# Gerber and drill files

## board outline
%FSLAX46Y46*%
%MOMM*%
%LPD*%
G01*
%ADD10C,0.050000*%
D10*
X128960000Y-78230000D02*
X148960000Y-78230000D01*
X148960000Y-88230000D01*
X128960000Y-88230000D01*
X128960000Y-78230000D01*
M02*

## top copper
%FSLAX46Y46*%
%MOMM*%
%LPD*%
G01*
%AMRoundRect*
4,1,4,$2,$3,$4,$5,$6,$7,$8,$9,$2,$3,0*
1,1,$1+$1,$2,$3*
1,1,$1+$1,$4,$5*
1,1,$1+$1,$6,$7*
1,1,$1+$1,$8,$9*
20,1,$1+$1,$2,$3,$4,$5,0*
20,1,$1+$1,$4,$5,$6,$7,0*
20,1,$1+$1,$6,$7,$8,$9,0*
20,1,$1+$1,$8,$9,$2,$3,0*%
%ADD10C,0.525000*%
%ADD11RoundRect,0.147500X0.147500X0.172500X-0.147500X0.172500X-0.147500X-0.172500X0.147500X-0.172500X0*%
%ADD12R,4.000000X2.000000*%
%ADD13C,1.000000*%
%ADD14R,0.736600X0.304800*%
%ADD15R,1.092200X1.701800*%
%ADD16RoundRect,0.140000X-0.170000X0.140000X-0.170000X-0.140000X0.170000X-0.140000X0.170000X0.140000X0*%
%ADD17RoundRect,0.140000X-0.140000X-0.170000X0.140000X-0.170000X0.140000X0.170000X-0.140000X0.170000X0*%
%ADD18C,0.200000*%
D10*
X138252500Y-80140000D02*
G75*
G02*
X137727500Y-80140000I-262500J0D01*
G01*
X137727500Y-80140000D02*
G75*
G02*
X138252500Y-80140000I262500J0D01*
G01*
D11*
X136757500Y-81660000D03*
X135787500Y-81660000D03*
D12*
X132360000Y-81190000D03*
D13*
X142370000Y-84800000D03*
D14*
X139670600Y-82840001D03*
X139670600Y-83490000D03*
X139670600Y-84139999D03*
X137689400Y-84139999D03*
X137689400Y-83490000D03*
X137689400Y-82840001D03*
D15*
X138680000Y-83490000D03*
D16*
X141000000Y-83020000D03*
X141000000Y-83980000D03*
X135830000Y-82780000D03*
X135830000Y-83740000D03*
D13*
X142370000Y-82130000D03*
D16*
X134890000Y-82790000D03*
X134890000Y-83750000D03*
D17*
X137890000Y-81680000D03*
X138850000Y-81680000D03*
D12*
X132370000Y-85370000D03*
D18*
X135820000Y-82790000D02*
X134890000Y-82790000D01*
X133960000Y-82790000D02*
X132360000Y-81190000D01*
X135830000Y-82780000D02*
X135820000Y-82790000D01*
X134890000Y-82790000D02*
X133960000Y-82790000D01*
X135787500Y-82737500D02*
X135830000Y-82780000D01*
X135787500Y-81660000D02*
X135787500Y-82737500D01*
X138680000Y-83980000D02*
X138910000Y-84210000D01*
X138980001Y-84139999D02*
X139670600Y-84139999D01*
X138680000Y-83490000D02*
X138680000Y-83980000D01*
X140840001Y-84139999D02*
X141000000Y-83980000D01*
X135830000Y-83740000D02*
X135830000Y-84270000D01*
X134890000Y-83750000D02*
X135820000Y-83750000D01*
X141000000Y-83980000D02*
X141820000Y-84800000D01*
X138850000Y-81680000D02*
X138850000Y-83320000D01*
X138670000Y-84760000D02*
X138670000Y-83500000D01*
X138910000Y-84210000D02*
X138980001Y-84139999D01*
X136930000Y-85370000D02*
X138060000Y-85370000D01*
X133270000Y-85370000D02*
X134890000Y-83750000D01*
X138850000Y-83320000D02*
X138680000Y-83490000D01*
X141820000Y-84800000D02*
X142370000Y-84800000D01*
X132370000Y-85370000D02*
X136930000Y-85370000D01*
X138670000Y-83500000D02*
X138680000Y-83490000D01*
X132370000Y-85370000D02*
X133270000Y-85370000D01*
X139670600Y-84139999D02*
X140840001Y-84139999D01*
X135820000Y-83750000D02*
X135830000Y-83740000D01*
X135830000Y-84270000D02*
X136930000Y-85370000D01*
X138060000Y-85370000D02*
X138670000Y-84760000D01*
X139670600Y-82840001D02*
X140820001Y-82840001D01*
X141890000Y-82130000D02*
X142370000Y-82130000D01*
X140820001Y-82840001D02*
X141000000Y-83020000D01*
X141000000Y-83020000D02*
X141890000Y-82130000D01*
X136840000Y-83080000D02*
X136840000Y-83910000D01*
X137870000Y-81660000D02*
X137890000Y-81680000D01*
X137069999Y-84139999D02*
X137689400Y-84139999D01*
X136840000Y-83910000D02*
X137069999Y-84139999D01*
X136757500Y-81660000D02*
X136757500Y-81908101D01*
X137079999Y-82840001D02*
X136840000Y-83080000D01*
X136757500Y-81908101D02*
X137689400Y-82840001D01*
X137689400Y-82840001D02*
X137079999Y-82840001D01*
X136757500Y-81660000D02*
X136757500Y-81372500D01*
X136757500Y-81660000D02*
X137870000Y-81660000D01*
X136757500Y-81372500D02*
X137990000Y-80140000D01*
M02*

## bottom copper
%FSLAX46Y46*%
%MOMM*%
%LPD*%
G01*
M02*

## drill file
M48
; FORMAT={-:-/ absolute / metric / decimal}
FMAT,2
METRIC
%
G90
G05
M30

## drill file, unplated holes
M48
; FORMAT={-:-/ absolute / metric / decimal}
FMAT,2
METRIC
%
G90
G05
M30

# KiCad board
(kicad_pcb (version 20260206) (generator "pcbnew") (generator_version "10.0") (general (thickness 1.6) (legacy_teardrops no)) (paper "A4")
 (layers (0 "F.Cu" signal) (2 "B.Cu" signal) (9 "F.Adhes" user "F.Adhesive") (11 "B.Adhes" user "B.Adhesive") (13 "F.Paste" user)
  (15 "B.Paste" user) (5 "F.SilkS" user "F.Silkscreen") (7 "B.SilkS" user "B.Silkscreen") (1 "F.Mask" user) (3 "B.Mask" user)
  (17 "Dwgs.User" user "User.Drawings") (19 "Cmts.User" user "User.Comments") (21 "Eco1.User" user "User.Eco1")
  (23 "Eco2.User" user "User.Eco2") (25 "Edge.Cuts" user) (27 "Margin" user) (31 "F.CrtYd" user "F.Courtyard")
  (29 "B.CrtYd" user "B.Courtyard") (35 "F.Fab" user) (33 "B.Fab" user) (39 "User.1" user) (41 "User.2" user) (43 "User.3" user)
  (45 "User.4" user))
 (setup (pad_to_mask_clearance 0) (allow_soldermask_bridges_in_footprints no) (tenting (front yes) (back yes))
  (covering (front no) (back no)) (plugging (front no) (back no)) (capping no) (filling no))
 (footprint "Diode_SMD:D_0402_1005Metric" (layer "F.Cu") (at 136.2725 81.66 180)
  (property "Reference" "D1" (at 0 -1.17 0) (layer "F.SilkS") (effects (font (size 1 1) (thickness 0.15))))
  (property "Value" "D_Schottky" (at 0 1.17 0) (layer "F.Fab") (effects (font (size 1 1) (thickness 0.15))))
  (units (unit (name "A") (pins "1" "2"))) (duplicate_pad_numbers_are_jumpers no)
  (pad "1" smd roundrect (at -0.485 0 180) (size 0.59 0.64) (layers "F.Cu" "F.Mask" "F.Paste") (roundrect_rratio 0.25) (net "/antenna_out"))
  (pad "2" smd roundrect (at 0.485 0 180) (size 0.59 0.64) (layers "F.Cu" "F.Mask" "F.Paste") (roundrect_rratio 0.25) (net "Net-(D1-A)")))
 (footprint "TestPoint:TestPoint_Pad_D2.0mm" (layer "F.Cu") (at 132.36 81.19)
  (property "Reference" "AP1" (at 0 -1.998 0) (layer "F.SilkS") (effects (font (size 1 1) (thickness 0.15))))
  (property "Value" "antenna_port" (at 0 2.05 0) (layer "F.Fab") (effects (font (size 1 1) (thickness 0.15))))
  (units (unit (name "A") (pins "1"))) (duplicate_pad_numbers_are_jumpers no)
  (pad "1" smd rect (at 0 0) (size 4 2) (layers "F.Cu" "F.Mask") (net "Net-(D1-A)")))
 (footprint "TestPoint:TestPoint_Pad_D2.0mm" (layer "F.Cu") (at 142.37 84.8)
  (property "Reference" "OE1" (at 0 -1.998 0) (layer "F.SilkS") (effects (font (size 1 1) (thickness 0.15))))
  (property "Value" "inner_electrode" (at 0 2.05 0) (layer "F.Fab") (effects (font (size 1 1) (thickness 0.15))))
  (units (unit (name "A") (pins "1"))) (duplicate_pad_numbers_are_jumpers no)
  (pad "1" smd circle (at 0 0) (size 1 1) (layers "F.Cu" "F.Mask") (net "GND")))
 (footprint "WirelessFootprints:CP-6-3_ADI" (layer "F.Cu") (at 138.68 83.49)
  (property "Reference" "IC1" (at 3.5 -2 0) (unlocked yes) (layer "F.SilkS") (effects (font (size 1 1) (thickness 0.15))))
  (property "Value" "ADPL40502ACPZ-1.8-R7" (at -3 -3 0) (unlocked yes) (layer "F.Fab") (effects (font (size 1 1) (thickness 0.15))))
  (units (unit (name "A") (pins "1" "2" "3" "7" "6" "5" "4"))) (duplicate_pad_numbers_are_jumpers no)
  (pad "1" smd rect (at 0.9906 -0.649999) (size 0.7366 0.3048) (layers "F.Cu" "F.Mask" "F.Paste") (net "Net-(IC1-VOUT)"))
  (pad "2" smd rect (at 0.9906 0) (size 0.7366 0.3048) (layers "F.Cu" "F.Mask" "F.Paste") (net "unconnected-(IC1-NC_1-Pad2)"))
  (pad "3" smd rect (at 0.9906 0.649999) (size 0.7366 0.3048) (layers "F.Cu" "F.Mask" "F.Paste") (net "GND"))
  (pad "4" smd rect (at -0.9906 0.649999) (size 0.7366 0.3048) (layers "F.Cu" "F.Mask" "F.Paste") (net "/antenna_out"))
  (pad "5" smd rect (at -0.9906 0) (size 0.7366 0.3048) (layers "F.Cu" "F.Mask" "F.Paste") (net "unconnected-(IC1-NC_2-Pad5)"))
  (pad "6" smd rect (at -0.9906 -0.649999) (size 0.7366 0.3048) (layers "F.Cu" "F.Mask" "F.Paste") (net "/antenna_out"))
  (pad "7" smd rect (at 0 0) (size 1.0922 1.7018) (layers "F.Cu" "F.Mask" "F.Paste") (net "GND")))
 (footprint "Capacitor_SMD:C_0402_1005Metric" (layer "F.Cu") (at 141 83.5 -90)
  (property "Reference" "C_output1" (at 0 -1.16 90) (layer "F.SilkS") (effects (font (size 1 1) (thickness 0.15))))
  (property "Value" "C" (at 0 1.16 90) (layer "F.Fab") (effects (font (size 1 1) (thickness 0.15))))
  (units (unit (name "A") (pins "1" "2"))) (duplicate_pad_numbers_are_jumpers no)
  (pad "1" smd roundrect (at -0.48 0 270) (size 0.56 0.62) (layers "F.Cu" "F.Mask" "F.Paste") (roundrect_rratio 0.25) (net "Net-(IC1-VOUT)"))
  (pad "2" smd roundrect (at 0.48 0 270) (size 0.56 0.62) (layers "F.Cu" "F.Mask" "F.Paste") (roundrect_rratio 0.25) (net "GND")))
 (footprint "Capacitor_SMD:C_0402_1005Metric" (layer "F.Cu") (at 135.83 83.26 -90)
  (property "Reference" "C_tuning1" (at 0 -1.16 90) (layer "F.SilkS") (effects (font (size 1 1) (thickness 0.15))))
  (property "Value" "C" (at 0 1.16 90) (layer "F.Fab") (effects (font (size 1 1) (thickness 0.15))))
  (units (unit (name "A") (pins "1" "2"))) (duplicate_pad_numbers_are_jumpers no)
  (pad "1" smd roundrect (at -0.48 0 270) (size 0.56 0.62) (layers "F.Cu" "F.Mask" "F.Paste") (roundrect_rratio 0.25) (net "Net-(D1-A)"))
  (pad "2" smd roundrect (at 0.48 0 270) (size 0.56 0.62) (layers "F.Cu" "F.Mask" "F.Paste") (roundrect_rratio 0.25) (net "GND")))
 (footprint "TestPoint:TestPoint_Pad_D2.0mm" (layer "F.Cu") (at 142.37 82.13)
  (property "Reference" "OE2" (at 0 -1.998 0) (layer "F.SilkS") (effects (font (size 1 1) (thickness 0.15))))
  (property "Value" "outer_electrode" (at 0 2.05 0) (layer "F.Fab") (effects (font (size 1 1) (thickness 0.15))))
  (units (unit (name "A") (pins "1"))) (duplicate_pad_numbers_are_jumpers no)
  (pad "1" smd circle (at 0 0) (size 1 1) (layers "F.Cu" "F.Mask") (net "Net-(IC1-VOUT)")))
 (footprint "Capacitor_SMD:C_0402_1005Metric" (layer "F.Cu") (at 134.89 83.27 -90)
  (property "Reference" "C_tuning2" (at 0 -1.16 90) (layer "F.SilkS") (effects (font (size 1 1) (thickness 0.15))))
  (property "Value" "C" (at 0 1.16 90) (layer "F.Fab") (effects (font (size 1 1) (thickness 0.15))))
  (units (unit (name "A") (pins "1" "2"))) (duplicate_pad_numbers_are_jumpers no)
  (pad "1" smd roundrect (at -0.48 0 270) (size 0.56 0.62) (layers "F.Cu" "F.Mask" "F.Paste") (roundrect_rratio 0.25) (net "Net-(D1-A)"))
  (pad "2" smd roundrect (at 0.48 0 270) (size 0.56 0.62) (layers "F.Cu" "F.Mask" "F.Paste") (roundrect_rratio 0.25) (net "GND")))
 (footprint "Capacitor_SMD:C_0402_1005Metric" (layer "F.Cu") (at 138.37 81.68)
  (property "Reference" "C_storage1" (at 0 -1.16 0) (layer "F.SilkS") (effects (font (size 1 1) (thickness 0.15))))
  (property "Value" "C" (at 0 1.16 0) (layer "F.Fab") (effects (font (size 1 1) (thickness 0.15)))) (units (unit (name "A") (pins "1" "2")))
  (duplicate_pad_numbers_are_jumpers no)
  (pad "1" smd roundrect (at -0.48 0) (size 0.56 0.62) (layers "F.Cu" "F.Mask" "F.Paste") (roundrect_rratio 0.25) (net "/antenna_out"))
  (pad "2" smd roundrect (at 0.48 0) (size 0.56 0.62) (layers "F.Cu" "F.Mask" "F.Paste") (roundrect_rratio 0.25) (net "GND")))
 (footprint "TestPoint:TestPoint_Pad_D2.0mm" (layer "F.Cu") (at 132.37 85.37)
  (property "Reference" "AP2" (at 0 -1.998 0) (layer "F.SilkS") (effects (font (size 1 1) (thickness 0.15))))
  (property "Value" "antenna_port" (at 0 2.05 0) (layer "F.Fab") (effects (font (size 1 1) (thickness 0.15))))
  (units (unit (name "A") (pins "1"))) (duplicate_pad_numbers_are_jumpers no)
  (pad "1" smd rect (at 0 0) (size 4 2) (layers "F.Cu" "F.Mask") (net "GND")))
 (gr_circle (center 137.99 80.14) (end 138.49 80.14) (stroke (width 0.05) (type solid)) (fill yes) (layer "F.Cu") (net "/antenna_out"))
 (gr_rect (start 128.96 78.23) (end 148.96 88.23) (stroke (width 0.05) (type solid)) (fill no) (layer "Edge.Cuts"))
 (segment (start 136.84 83.08) (end 136.84 83.91) (width 0.2) (layer "F.Cu") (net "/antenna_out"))
 (segment (start 137.87 81.66) (end 137.89 81.68) (width 0.2) (layer "F.Cu") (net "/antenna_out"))
 (segment (start 137.069999 84.139999) (end 137.6894 84.139999) (width 0.2) (layer "F.Cu") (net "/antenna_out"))
 (segment (start 136.84 83.91) (end 137.069999 84.139999) (width 0.2) (layer "F.Cu") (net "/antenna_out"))
 (segment (start 136.7575 81.66) (end 136.7575 81.908101) (width 0.2) (layer "F.Cu") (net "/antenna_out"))
 (segment (start 137.079999 82.840001) (end 136.84 83.08) (width 0.2) (layer "F.Cu") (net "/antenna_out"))
 (segment (start 136.7575 81.908101) (end 137.6894 82.840001) (width 0.2) (layer "F.Cu") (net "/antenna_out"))
 (segment (start 137.6894 82.840001) (end 137.079999 82.840001) (width 0.2) (layer "F.Cu") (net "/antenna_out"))
 (segment (start 136.7575 81.66) (end 136.7575 81.3725) (width 0.2) (layer "F.Cu") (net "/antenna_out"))
 (segment (start 136.7575 81.66) (end 137.87 81.66) (width 0.2) (layer "F.Cu") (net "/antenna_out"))
 (segment (start 136.7575 81.3725) (end 137.99 80.14) (width 0.2) (layer "F.Cu") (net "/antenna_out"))
 (segment (start 135.82 82.79) (end 134.89 82.79) (width 0.2) (layer "F.Cu") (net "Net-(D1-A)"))
 (segment (start 133.96 82.79) (end 132.36 81.19) (width 0.2) (layer "F.Cu") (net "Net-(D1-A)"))
 (segment (start 135.83 82.78) (end 135.82 82.79) (width 0.2) (layer "F.Cu") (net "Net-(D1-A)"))
 (segment (start 134.89 82.79) (end 133.96 82.79) (width 0.2) (layer "F.Cu") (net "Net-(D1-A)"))
 (segment (start 135.7875 82.7375) (end 135.83 82.78) (width 0.2) (layer "F.Cu") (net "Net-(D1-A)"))
 (segment (start 135.7875 81.66) (end 135.7875 82.7375) (width 0.2) (layer "F.Cu") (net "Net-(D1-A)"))
 (segment (start 138.68 83.98) (end 138.91 84.21) (width 0.2) (layer "F.Cu") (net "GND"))
 (segment (start 138.980001 84.139999) (end 139.6706 84.139999) (width 0.2) (layer "F.Cu") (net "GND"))
 (segment (start 138.68 83.49) (end 138.68 83.98) (width 0.2) (layer "F.Cu") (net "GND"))
 (segment (start 140.840001 84.139999) (end 141 83.98) (width 0.2) (layer "F.Cu") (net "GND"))
 (segment (start 135.83 83.74) (end 135.83 84.27) (width 0.2) (layer "F.Cu") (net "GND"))
 (segment (start 134.89 83.75) (end 135.82 83.75) (width 0.2) (layer "F.Cu") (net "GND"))
 (segment (start 141 83.98) (end 141.82 84.8) (width 0.2) (layer "F.Cu") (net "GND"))
 (segment (start 138.85 81.68) (end 138.85 83.32) (width 0.2) (layer "F.Cu") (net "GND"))
 (segment (start 138.67 84.76) (end 138.67 83.5) (width 0.2) (layer "F.Cu") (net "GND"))
 (segment (start 138.91 84.21) (end 138.980001 84.139999) (width 0.2) (layer "F.Cu") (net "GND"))
 (segment (start 136.93 85.37) (end 138.06 85.37) (width 0.2) (layer "F.Cu") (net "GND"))
 (segment (start 133.27 85.37) (end 134.89 83.75) (width 0.2) (layer "F.Cu") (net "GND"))
 (segment (start 138.85 83.32) (end 138.68 83.49) (width 0.2) (layer "F.Cu") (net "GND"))
 (segment (start 141.82 84.8) (end 142.37 84.8) (width 0.2) (layer "F.Cu") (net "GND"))
 (segment (start 132.37 85.37) (end 136.93 85.37) (width 0.2) (layer "F.Cu") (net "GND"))
 (segment (start 138.67 83.5) (end 138.68 83.49) (width 0.2) (layer "F.Cu") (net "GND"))
 (segment (start 132.37 85.37) (end 133.27 85.37) (width 0.2) (layer "F.Cu") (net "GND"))
 (segment (start 139.6706 84.139999) (end 140.840001 84.139999) (width 0.2) (layer "F.Cu") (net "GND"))
 (segment (start 135.82 83.75) (end 135.83 83.74) (width 0.2) (layer "F.Cu") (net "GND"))
 (segment (start 135.83 84.27) (end 136.93 85.37) (width 0.2) (layer "F.Cu") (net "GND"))
 (segment (start 138.06 85.37) (end 138.67 84.76) (width 0.2) (layer "F.Cu") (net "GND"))
 (segment (start 139.6706 82.840001) (end 140.820001 82.840001) (width 0.2) (layer "F.Cu") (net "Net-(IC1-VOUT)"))
 (segment (start 141.89 82.13) (end 142.37 82.13) (width 0.2) (layer "F.Cu") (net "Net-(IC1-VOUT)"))
 (segment (start 140.820001 82.840001) (end 141 83.02) (width 0.2) (layer "F.Cu") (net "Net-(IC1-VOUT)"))
 (segment (start 141 83.02) (end 141.89 82.13) (width 0.2) (layer "F.Cu") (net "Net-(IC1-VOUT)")))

